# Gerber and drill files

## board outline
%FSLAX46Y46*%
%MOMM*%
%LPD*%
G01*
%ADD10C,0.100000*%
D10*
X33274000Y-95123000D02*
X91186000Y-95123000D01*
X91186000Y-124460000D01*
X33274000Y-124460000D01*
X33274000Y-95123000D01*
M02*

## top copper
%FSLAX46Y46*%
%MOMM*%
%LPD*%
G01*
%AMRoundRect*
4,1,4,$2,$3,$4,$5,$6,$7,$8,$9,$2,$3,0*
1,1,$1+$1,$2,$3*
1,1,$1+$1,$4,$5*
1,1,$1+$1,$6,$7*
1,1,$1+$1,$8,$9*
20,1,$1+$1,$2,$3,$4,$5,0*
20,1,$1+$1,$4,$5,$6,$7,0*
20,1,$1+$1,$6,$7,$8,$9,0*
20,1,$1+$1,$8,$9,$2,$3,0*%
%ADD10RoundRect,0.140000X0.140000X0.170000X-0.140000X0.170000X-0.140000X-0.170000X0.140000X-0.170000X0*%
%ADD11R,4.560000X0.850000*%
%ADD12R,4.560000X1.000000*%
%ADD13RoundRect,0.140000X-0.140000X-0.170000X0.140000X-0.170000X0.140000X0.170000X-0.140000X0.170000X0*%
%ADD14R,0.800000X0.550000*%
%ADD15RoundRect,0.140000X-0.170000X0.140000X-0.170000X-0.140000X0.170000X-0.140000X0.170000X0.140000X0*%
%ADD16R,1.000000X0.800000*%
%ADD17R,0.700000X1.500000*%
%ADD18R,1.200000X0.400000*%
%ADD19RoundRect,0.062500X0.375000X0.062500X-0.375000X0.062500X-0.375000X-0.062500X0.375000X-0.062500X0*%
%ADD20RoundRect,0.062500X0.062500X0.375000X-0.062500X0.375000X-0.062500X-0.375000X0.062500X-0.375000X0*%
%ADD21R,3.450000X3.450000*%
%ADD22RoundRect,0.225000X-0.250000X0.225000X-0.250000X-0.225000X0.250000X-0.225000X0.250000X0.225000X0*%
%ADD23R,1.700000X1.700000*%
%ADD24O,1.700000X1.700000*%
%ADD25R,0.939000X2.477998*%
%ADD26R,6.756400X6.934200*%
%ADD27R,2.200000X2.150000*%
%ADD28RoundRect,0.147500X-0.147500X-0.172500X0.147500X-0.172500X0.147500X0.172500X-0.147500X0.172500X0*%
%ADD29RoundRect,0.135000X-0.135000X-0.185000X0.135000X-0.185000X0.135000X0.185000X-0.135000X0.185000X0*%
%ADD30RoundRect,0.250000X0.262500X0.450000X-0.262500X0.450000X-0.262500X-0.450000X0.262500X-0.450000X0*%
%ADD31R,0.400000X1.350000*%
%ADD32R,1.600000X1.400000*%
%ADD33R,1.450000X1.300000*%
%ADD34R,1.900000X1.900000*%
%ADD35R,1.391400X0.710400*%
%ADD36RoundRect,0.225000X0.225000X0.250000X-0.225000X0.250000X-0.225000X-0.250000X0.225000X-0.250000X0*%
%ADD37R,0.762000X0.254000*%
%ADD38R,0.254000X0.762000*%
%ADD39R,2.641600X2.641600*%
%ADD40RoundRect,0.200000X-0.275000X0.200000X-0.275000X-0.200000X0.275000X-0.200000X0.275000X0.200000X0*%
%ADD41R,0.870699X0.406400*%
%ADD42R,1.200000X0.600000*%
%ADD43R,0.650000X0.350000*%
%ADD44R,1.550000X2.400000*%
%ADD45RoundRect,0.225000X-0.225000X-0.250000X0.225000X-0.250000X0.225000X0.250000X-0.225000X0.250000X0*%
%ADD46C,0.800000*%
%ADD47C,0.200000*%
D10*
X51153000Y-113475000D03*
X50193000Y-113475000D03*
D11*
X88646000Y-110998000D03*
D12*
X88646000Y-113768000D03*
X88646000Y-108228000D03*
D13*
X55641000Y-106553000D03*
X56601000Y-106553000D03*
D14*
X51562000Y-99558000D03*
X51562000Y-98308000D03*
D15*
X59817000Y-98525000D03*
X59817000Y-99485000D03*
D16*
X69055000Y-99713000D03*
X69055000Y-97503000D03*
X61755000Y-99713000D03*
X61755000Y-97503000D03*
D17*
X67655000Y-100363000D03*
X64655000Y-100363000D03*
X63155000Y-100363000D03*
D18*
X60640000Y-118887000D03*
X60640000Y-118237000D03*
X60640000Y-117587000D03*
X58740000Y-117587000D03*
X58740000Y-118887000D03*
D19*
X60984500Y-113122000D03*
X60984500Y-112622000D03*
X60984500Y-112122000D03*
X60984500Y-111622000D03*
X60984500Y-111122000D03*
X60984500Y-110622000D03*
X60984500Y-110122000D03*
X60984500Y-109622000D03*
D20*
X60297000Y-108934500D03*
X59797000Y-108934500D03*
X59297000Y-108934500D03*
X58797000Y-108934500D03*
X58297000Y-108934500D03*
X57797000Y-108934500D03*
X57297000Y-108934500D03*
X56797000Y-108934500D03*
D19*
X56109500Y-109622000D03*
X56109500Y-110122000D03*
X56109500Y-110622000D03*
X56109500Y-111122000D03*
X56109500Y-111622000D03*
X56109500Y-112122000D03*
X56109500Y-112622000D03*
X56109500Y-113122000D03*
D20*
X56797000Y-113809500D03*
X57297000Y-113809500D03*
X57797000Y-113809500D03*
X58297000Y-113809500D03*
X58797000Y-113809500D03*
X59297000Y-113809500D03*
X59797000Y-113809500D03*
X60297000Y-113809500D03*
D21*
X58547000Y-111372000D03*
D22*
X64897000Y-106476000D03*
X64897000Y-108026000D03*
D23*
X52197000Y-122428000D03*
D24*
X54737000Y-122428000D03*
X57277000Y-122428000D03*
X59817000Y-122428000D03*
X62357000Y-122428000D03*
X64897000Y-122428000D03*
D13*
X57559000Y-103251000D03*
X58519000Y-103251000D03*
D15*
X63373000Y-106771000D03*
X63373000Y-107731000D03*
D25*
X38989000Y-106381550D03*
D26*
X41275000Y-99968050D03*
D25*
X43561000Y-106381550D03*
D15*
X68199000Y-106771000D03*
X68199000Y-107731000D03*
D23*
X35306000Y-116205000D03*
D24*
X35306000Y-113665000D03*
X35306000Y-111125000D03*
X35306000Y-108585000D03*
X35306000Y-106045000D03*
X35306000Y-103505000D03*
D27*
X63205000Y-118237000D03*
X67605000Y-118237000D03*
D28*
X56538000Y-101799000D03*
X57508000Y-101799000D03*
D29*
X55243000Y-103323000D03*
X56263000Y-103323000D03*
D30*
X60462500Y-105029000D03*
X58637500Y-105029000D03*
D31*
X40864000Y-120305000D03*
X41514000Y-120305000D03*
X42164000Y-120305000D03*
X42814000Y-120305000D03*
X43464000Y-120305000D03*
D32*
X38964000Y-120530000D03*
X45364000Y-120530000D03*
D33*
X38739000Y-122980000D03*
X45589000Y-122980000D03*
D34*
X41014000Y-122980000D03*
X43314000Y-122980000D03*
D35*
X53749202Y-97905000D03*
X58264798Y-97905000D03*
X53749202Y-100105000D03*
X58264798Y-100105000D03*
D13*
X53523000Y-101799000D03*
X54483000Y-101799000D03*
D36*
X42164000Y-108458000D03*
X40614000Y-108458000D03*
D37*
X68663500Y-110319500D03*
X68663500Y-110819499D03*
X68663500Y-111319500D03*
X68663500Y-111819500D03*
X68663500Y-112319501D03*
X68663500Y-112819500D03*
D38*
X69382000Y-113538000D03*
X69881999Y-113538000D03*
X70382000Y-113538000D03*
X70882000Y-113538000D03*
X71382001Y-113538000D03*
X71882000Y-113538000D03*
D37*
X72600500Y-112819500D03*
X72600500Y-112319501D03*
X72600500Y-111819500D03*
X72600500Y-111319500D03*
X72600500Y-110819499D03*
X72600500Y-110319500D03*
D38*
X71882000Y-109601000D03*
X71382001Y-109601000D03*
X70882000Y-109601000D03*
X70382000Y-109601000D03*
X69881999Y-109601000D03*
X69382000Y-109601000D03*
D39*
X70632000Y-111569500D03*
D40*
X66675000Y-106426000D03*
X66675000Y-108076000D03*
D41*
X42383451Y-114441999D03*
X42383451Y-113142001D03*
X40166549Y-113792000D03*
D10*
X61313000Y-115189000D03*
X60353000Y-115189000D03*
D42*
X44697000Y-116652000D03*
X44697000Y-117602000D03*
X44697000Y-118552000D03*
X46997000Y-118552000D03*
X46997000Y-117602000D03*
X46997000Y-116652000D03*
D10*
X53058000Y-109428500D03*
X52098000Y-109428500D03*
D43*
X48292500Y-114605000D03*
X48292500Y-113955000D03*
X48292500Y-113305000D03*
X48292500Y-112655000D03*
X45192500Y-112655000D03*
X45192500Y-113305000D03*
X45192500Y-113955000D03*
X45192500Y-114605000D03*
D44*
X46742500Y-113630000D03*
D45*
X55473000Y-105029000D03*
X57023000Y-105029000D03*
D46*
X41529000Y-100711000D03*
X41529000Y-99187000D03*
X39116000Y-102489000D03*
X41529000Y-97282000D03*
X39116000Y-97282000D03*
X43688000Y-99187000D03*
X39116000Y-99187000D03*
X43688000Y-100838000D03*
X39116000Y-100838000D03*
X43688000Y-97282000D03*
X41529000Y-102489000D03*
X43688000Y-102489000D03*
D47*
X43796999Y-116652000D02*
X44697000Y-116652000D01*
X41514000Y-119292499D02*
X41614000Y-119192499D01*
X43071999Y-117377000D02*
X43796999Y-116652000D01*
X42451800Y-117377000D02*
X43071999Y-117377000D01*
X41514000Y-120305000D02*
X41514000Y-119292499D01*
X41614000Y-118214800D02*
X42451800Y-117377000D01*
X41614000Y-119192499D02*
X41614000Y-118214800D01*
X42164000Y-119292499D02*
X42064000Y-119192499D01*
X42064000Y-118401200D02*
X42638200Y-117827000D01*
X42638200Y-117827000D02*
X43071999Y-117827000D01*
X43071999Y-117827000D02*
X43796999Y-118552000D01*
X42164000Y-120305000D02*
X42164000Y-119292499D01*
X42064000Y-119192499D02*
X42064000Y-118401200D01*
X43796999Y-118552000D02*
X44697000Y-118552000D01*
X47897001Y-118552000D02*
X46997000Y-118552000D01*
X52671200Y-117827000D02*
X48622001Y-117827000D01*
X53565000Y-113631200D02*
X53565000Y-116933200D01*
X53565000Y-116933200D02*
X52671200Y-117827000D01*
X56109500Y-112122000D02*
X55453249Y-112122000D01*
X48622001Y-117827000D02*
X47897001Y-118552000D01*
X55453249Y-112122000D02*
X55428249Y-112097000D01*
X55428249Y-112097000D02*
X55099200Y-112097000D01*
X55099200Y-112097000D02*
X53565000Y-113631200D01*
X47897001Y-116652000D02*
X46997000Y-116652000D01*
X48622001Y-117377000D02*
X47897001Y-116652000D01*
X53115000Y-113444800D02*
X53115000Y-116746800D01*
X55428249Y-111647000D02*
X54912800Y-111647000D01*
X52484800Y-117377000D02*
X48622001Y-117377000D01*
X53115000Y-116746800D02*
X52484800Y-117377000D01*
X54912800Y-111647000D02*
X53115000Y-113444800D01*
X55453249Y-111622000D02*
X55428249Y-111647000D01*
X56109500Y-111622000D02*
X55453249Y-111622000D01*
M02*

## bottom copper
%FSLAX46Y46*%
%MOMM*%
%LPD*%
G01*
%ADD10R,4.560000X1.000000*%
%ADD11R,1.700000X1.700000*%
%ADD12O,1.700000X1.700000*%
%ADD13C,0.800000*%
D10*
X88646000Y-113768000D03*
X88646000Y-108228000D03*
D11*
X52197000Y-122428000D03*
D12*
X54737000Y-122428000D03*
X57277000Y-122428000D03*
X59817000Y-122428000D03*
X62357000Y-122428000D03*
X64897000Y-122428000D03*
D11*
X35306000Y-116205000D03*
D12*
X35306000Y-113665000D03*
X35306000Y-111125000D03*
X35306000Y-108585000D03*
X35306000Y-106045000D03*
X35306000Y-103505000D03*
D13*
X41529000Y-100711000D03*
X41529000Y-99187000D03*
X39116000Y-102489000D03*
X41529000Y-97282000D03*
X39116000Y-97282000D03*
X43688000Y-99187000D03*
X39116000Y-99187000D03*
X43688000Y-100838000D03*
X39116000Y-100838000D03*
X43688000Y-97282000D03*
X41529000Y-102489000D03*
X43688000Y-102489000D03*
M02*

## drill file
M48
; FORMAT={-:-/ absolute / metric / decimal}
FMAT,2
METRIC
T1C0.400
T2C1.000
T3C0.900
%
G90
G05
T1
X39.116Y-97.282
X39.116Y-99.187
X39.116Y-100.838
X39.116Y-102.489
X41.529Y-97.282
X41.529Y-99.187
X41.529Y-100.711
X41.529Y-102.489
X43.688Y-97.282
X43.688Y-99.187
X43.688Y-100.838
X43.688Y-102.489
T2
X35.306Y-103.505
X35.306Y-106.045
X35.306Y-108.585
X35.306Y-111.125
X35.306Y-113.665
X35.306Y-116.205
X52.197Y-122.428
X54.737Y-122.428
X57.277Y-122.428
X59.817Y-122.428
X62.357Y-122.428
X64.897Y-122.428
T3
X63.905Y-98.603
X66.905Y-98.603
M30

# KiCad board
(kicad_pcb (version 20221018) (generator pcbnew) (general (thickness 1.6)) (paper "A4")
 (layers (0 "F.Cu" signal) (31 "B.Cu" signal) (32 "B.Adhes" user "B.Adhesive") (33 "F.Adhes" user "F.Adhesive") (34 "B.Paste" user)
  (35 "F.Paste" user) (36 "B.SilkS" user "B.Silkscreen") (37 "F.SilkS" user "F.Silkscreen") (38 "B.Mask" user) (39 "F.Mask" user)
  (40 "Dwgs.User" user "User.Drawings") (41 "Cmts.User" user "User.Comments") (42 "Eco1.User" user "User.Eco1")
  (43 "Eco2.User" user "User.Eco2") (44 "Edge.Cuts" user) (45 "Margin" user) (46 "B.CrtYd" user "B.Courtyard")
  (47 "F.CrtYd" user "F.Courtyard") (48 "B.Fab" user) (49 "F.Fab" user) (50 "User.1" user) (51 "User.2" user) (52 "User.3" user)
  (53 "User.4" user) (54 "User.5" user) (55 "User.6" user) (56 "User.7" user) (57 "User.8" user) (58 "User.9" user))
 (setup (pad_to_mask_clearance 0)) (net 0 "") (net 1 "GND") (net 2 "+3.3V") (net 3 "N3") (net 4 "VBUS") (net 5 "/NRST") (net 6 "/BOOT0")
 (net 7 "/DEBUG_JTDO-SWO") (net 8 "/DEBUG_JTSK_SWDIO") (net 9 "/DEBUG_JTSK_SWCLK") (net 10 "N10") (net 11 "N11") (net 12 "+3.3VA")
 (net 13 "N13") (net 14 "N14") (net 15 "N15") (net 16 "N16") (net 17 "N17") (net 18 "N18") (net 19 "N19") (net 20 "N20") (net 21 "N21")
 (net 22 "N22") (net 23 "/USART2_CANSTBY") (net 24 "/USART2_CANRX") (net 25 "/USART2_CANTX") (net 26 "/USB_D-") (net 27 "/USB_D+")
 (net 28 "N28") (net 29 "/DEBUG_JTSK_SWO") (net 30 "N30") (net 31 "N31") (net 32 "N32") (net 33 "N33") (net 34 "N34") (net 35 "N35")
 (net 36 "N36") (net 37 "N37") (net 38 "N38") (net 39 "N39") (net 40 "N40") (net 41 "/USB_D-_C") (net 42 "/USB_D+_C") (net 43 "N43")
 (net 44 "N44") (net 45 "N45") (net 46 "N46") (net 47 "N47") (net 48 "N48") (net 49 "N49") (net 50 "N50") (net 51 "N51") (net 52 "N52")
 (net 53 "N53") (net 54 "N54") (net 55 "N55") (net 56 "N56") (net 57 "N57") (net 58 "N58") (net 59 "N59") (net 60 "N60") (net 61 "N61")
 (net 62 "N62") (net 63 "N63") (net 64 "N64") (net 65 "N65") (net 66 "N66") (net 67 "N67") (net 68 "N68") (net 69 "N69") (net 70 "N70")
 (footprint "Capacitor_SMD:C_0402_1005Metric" (layer "F.Cu") (at 50.673 113.475 180)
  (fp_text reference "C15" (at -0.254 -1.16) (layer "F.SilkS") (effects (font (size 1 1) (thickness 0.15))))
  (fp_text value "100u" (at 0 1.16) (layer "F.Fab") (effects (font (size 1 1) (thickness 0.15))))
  (pad "1" smd roundrect (at -0.48 0 180) (size 0.56 0.62) (layers "F.Cu" "F.Paste" "F.Mask") (roundrect_rratio 0.25) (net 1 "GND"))
  (pad "2" smd roundrect (at 0.48 0 180) (size 0.56 0.62) (layers "F.Cu" "F.Paste" "F.Mask") (roundrect_rratio 0.25) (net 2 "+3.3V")))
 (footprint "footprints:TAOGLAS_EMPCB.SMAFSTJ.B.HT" (layer "F.Cu") (at 88.646 110.998 90)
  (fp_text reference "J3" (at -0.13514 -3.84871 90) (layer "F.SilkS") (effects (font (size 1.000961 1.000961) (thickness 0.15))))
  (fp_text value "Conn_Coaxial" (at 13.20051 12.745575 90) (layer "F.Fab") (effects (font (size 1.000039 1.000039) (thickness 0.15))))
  (pad "1" smd rect (at 0 0 90) (size 0.85 4.56) (layers "F.Cu" "F.Paste" "F.Mask") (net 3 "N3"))
  (pad "SH1" smd rect (at -2.77 0 90) (size 1 4.56) (layers "F.Cu" "F.Paste" "F.Mask"))
  (pad "SH2" smd rect (at 2.77 0 90) (size 1 4.56) (layers "F.Cu" "F.Paste" "F.Mask"))
  (pad "SH3" smd rect (at -2.77 0 90) (size 1 4.56) (layers "B.Cu" "B.Paste" "B.Mask"))
  (pad "SH4" smd rect (at 2.77 0 90) (size 1 4.56) (layers "B.Cu" "B.Paste" "B.Mask")))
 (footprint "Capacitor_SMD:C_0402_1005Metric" (layer "F.Cu") (at 56.121 106.553)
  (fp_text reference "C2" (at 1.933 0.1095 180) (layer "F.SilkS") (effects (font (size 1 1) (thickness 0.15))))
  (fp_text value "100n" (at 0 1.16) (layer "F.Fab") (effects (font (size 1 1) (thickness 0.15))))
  (pad "1" smd roundrect (at -0.48 0) (size 0.56 0.62) (layers "F.Cu" "F.Paste" "F.Mask") (roundrect_rratio 0.25) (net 2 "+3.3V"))
  (pad "2" smd roundrect (at 0.48 0) (size 0.56 0.62) (layers "F.Cu" "F.Paste" "F.Mask") (roundrect_rratio 0.25) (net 1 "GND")))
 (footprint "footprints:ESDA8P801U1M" (layer "F.Cu") (at 51.562 98.933 90)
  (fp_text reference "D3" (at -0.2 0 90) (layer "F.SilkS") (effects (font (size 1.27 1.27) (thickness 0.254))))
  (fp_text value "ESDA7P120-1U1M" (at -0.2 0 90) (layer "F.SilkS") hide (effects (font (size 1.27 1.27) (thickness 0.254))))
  (pad "1" smd rect (at -0.625 0 90) (size 0.55 0.8) (layers "F.Cu" "F.Paste" "F.Mask") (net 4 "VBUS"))
  (pad "2" smd rect (at 0.625 0 90) (size 0.55 0.8) (layers "F.Cu" "F.Paste" "F.Mask") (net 1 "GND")))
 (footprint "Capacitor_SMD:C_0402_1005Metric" (layer "F.Cu") (at 59.817 99.005 -90)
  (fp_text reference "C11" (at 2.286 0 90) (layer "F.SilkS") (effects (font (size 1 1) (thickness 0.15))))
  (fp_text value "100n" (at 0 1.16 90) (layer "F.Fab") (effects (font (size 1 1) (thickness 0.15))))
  (pad "1" smd roundrect (at -0.48 0 270) (size 0.56 0.62) (layers "F.Cu" "F.Paste" "F.Mask") (roundrect_rratio 0.25) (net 1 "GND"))
  (pad "2" smd roundrect (at 0.48 0 270) (size 0.56 0.62) (layers "F.Cu" "F.Paste" "F.Mask") (roundrect_rratio 0.25) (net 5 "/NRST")))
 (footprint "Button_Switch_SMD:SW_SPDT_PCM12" (layer "F.Cu") (at 65.405 98.933 180)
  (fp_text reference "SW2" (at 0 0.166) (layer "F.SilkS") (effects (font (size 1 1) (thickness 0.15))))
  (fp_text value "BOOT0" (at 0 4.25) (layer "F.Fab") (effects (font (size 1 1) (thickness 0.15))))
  (pad "" smd rect (at -3.65 -0.78 180) (size 1 0.8) (layers "F.Cu" "F.Paste" "F.Mask"))
  (pad "" smd rect (at -3.65 1.43 180) (size 1 0.8) (layers "F.Cu" "F.Paste" "F.Mask"))
  (pad "" np_thru_hole circle (at -1.5 0.33 180) (size 0.9 0.9) (drill 0.9) (layers "*.Cu" "*.Mask"))
  (pad "" np_thru_hole circle (at 1.5 0.33 180) (size 0.9 0.9) (drill 0.9) (layers "*.Cu" "*.Mask"))
  (pad "" smd rect (at 3.65 -0.78 180) (size 1 0.8) (layers "F.Cu" "F.Paste" "F.Mask"))
  (pad "" smd rect (at 3.65 1.43 180) (size 1 0.8) (layers "F.Cu" "F.Paste" "F.Mask"))
  (pad "1" smd rect (at -2.25 -1.43 180) (size 0.7 1.5) (layers "F.Cu" "F.Paste" "F.Mask") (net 1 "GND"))
  (pad "2" smd rect (at 0.75 -1.43 180) (size 0.7 1.5) (layers "F.Cu" "F.Paste" "F.Mask") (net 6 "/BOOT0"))
  (pad "3" smd rect (at 2.25 -1.43 180) (size 0.7 1.5) (layers "F.Cu" "F.Paste" "F.Mask") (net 2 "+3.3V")))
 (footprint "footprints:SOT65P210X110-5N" (layer "F.Cu") (at 59.69 118.237 180)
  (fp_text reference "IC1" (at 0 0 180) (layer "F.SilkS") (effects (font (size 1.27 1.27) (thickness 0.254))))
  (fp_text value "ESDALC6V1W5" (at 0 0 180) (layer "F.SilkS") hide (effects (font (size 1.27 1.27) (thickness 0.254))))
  (pad "1" smd rect (at -0.95 -0.65 270) (size 0.4 1.2) (layers "F.Cu" "F.Paste" "F.Mask") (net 5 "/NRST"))
  (pad "2" smd rect (at -0.95 0 270) (size 0.4 1.2) (layers "F.Cu" "F.Paste" "F.Mask") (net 1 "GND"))
  (pad "3" smd rect (at -0.95 0.65 270) (size 0.4 1.2) (layers "F.Cu" "F.Paste" "F.Mask") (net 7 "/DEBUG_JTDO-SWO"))
  (pad "4" smd rect (at 0.95 0.65 270) (size 0.4 1.2) (layers "F.Cu" "F.Paste" "F.Mask") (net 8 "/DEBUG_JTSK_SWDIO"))
  (pad "5" smd rect (at 0.95 -0.65 270) (size 0.4 1.2) (layers "F.Cu" "F.Paste" "F.Mask") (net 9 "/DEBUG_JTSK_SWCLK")))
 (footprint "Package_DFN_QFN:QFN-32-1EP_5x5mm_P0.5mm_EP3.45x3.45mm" (layer "F.Cu") (at 58.547 111.372 180)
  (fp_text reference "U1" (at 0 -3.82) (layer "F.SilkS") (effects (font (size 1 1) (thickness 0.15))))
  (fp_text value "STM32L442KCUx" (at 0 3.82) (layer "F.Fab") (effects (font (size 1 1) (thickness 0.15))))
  (pad "" smd roundrect (at -1.15 -1.15 180) (size 0.93 0.93) (layers "F.Paste") (roundrect_rratio 0.25))
  (pad "" smd roundrect (at -1.15 0 180) (size 0.93 0.93) (layers "F.Paste") (roundrect_rratio 0.25))
  (pad "" smd roundrect (at -1.15 1.15 180) (size 0.93 0.93) (layers "F.Paste") (roundrect_rratio 0.25))
  (pad "" smd roundrect (at 0 -1.15 180) (size 0.93 0.93) (layers "F.Paste") (roundrect_rratio 0.25))
  (pad "" smd roundrect (at 0 0 180) (size 0.93 0.93) (layers "F.Paste") (roundrect_rratio 0.25))
  (pad "" smd roundrect (at 0 1.15 180) (size 0.93 0.93) (layers "F.Paste") (roundrect_rratio 0.25))
  (pad "" smd roundrect (at 1.15 -1.15 180) (size 0.93 0.93) (layers "F.Paste") (roundrect_rratio 0.25))
  (pad "" smd roundrect (at 1.15 0 180) (size 0.93 0.93) (layers "F.Paste") (roundrect_rratio 0.25))
  (pad "" smd roundrect (at 1.15 1.15 180) (size 0.93 0.93) (layers "F.Paste") (roundrect_rratio 0.25))
  (pad "1" smd roundrect (at -2.4375 -1.75 180) (size 0.875 0.25) (layers "F.Cu" "F.Paste" "F.Mask") (roundrect_rratio 0.25) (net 2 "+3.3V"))
  (pad "2" smd roundrect (at -2.4375 -1.25 180) (size 0.875 0.25) (layers "F.Cu" "F.Paste" "F.Mask") (roundrect_rratio 0.25) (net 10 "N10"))
  (pad "3" smd roundrect (at -2.4375 -0.75 180) (size 0.875 0.25) (layers "F.Cu" "F.Paste" "F.Mask") (roundrect_rratio 0.25) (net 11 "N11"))
  (pad "4" smd roundrect (at -2.4375 -0.25 180) (size 0.875 0.25) (layers "F.Cu" "F.Paste" "F.Mask") (roundrect_rratio 0.25) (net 5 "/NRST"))
  (pad "5" smd roundrect (at -2.4375 0.25 180) (size 0.875 0.25) (layers "F.Cu" "F.Paste" "F.Mask") (roundrect_rratio 0.25)
   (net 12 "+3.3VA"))
  (pad "6" smd roundrect (at -2.4375 0.75 180) (size 0.875 0.25) (layers "F.Cu" "F.Paste" "F.Mask") (roundrect_rratio 0.25) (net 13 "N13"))
  (pad "7" smd roundrect (at -2.4375 1.25 180) (size 0.875 0.25) (layers "F.Cu" "F.Paste" "F.Mask") (roundrect_rratio 0.25) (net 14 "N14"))
  (pad "8" smd roundrect (at -2.4375 1.75 180) (size 0.875 0.25) (layers "F.Cu" "F.Paste" "F.Mask") (roundrect_rratio 0.25) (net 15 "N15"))
  (pad "9" smd roundrect (at -1.75 2.4375 180) (size 0.25 0.875) (layers "F.Cu" "F.Paste" "F.Mask") (roundrect_rratio 0.25) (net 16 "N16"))
  (pad "10" smd roundrect (at -1.25 2.4375 180) (size 0.25 0.875) (layers "F.Cu" "F.Paste" "F.Mask") (roundrect_rratio 0.25) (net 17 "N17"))
  (pad "11" smd roundrect (at -0.75 2.4375 180) (size 0.25 0.875) (layers "F.Cu" "F.Paste" "F.Mask") (roundrect_rratio 0.25) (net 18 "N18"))
  (pad "12" smd roundrect (at -0.25 2.4375 180) (size 0.25 0.875) (layers "F.Cu" "F.Paste" "F.Mask") (roundrect_rratio 0.25) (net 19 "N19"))
  (pad "13" smd roundrect (at 0.25 2.4375 180) (size 0.25 0.875) (layers "F.Cu" "F.Paste" "F.Mask") (roundrect_rratio 0.25) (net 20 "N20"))
  (pad "14" smd roundrect (at 0.75 2.4375 180) (size 0.25 0.875) (layers "F.Cu" "F.Paste" "F.Mask") (roundrect_rratio 0.25) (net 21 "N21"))
  (pad "15" smd roundrect (at 1.25 2.4375 180) (size 0.25 0.875) (layers "F.Cu" "F.Paste" "F.Mask") (roundrect_rratio 0.25) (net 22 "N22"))
  (pad "16" smd roundrect (at 1.75 2.4375 180) (size 0.25 0.875) (layers "F.Cu" "F.Paste" "F.Mask") (roundrect_rratio 0.25) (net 1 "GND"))
  (pad "17" smd roundrect (at 2.4375 1.75 180) (size 0.875 0.25) (layers "F.Cu" "F.Paste" "F.Mask") (roundrect_rratio 0.25) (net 2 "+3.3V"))
  (pad "18" smd roundrect (at 2.4375 1.25 180) (size 0.875 0.25) (layers "F.Cu" "F.Paste" "F.Mask") (roundrect_rratio 0.25)
   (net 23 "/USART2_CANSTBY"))
  (pad "19" smd roundrect (at 2.4375 0.75 180) (size 0.875 0.25) (layers "F.Cu" "F.Paste" "F.Mask") (roundrect_rratio 0.25)
   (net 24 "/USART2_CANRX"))
  (pad "20" smd roundrect (at 2.4375 0.25 180) (size 0.875 0.25) (layers "F.Cu" "F.Paste" "F.Mask") (roundrect_rratio 0.25)
   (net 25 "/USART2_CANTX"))
  (pad "21" smd roundrect (at 2.4375 -0.25 180) (size 0.875 0.25) (layers "F.Cu" "F.Paste" "F.Mask") (roundrect_rratio 0.25)
   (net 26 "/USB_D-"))
  (pad "22" smd roundrect (at 2.4375 -0.75 180) (size 0.875 0.25) (layers "F.Cu" "F.Paste" "F.Mask") (roundrect_rratio 0.25)
   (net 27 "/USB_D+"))
  (pad "23" smd roundrect (at 2.4375 -1.25 180) (size 0.875 0.25) (layers "F.Cu" "F.Paste" "F.Mask") (roundrect_rratio 0.25)
   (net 8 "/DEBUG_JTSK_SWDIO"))
  (pad "24" smd roundrect (at 2.4375 -1.75 180) (size 0.875 0.25) (layers "F.Cu" "F.Paste" "F.Mask") (roundrect_rratio 0.25)
   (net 9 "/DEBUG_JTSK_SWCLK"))
  (pad "25" smd roundrect (at 1.75 -2.4375 180) (size 0.25 0.875) (layers "F.Cu" "F.Paste" "F.Mask") (roundrect_rratio 0.25) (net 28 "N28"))
  (pad "26" smd roundrect (at 1.25 -2.4375 180) (size 0.25 0.875) (layers "F.Cu" "F.Paste" "F.Mask") (roundrect_rratio 0.25)
   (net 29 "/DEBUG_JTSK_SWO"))
  (pad "27" smd roundrect (at 0.75 -2.4375 180) (size 0.25 0.875) (layers "F.Cu" "F.Paste" "F.Mask") (roundrect_rratio 0.25) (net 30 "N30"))
  (pad "28" smd roundrect (at 0.25 -2.4375 180) (size 0.25 0.875) (layers "F.Cu" "F.Paste" "F.Mask") (roundrect_rratio 0.25) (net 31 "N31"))
  (pad "29" smd roundrect (at -0.25 -2.4375 180) (size 0.25 0.875) (layers "F.Cu" "F.Paste" "F.Mask") (roundrect_rratio 0.25) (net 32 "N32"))
  (pad "30" smd roundrect (at -0.75 -2.4375 180) (size 0.25 0.875) (layers "F.Cu" "F.Paste" "F.Mask") (roundrect_rratio 0.25) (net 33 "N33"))
  (pad "31" smd roundrect (at -1.25 -2.4375 180) (size 0.25 0.875) (layers "F.Cu" "F.Paste" "F.Mask") (roundrect_rratio 0.25)
   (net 6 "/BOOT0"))
  (pad "32" smd roundrect (at -1.75 -2.4375 180) (size 0.25 0.875) (layers "F.Cu" "F.Paste" "F.Mask") (roundrect_rratio 0.25) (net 1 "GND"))
  (pad "33" smd rect (at 0 0 180) (size 3.45 3.45) (layers "F.Cu" "F.Mask") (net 1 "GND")))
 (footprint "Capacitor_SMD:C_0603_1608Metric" (layer "F.Cu") (at 64.897 107.251 -90)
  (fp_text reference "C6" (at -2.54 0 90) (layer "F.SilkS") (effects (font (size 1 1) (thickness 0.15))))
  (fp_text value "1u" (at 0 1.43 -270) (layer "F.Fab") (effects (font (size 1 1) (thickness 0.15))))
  (pad "1" smd roundrect (at -0.775 0 270) (size 0.9 0.95) (layers "F.Cu" "F.Paste" "F.Mask") (roundrect_rratio 0.25) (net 12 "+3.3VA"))
  (pad "2" smd roundrect (at 0.775 0 270) (size 0.9 0.95) (layers "F.Cu" "F.Paste" "F.Mask") (roundrect_rratio 0.25) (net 1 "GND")))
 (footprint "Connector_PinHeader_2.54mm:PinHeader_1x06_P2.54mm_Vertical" (layer "F.Cu") (at 52.197 122.428 90)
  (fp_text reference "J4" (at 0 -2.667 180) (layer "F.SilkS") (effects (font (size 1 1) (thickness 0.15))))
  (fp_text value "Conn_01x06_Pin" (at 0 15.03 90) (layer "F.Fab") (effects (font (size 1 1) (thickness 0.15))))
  (pad "1" thru_hole rect (at 0 0 90) (size 1.7 1.7) (drill 1) (layers "*.Cu" "*.Mask") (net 2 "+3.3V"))
  (pad "2" thru_hole oval (at 0 2.54 90) (size 1.7 1.7) (drill 1) (layers "*.Cu" "*.Mask") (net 9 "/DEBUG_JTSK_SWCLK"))
  (pad "3" thru_hole oval (at 0 5.08 90) (size 1.7 1.7) (drill 1) (layers "*.Cu" "*.Mask") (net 1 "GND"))
  (pad "4" thru_hole oval (at 0 7.62 90) (size 1.7 1.7) (drill 1) (layers "*.Cu" "*.Mask") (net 8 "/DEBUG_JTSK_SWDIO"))
  (pad "5" thru_hole oval (at 0 10.16 90) (size 1.7 1.7) (drill 1) (layers "*.Cu" "*.Mask") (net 5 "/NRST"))
  (pad "6" thru_hole oval (at 0 12.7 90) (size 1.7 1.7) (drill 1) (layers "*.Cu" "*.Mask") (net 7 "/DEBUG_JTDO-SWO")))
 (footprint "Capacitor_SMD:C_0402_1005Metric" (layer "F.Cu") (at 58.039 103.251)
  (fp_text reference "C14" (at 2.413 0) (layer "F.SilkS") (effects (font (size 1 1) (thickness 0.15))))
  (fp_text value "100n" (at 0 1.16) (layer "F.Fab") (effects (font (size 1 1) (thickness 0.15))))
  (pad "1" smd roundrect (at -0.48 0) (size 0.56 0.62) (layers "F.Cu" "F.Paste" "F.Mask") (roundrect_rratio 0.25) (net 1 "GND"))
  (pad "2" smd roundrect (at 0.48 0) (size 0.56 0.62) (layers "F.Cu" "F.Paste" "F.Mask") (roundrect_rratio 0.25) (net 4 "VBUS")))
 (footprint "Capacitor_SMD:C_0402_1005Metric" (layer "F.Cu") (at 63.373 107.251 -90)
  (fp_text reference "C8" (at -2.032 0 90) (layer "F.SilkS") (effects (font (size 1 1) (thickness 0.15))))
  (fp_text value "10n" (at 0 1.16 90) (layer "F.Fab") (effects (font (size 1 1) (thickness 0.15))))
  (pad "1" smd roundrect (at -0.48 0 270) (size 0.56 0.62) (layers "F.Cu" "F.Paste" "F.Mask") (roundrect_rratio 0.25) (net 12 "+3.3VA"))
  (pad "2" smd roundrect (at 0.48 0 270) (size 0.56 0.62) (layers "F.Cu" "F.Paste" "F.Mask") (roundrect_rratio 0.25) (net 1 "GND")))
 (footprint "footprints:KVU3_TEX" (layer "F.Cu") (at 41.275 99.96805)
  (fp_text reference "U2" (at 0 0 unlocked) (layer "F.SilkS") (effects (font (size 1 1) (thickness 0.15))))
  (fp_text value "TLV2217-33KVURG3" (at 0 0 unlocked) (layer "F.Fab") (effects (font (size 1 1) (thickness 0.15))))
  (pad "1" smd rect (at -2.286 6.4135) (size 0.939 2.477998) (layers "F.Cu" "F.Paste" "F.Mask") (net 2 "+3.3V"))
  (pad "2" smd rect (at 0 0) (size 6.7564 6.9342) (layers "F.Cu" "F.Paste" "F.Mask") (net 1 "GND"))
  (pad "3" smd rect (at 2.286 6.4135) (size 0.939 2.477998) (layers "F.Cu" "F.Paste" "F.Mask") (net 4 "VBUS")))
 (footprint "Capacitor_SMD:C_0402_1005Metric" (layer "F.Cu") (at 68.199 107.251 -90)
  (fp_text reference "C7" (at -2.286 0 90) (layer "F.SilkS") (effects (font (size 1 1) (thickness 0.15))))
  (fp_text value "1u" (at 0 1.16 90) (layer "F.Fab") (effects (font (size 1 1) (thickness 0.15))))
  (pad "1" smd roundrect (at -0.48 0 270) (size 0.56 0.62) (layers "F.Cu" "F.Paste" "F.Mask") (roundrect_rratio 0.25) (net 2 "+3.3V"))
  (pad "2" smd roundrect (at 0.48 0 270) (size 0.56 0.62) (layers "F.Cu" "F.Paste" "F.Mask") (roundrect_rratio 0.25) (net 1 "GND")))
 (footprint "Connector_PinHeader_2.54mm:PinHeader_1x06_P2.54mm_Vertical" (layer "F.Cu") (at 35.306 116.205 180)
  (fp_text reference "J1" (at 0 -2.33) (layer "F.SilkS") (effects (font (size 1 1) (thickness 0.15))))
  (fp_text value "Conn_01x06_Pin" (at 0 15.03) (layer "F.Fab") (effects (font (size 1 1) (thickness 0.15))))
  (pad "1" thru_hole rect (at 0 0 180) (size 1.7 1.7) (drill 1) (layers "*.Cu" "*.Mask") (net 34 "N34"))
  (pad "2" thru_hole oval (at 0 2.54 180) (size 1.7 1.7) (drill 1) (layers "*.Cu" "*.Mask") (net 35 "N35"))
  (pad "3" thru_hole oval (at 0 5.08 180) (size 1.7 1.7) (drill 1) (layers "*.Cu" "*.Mask") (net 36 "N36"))
  (pad "4" thru_hole oval (at 0 7.62 180) (size 1.7 1.7) (drill 1) (layers "*.Cu" "*.Mask") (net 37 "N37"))
  (pad "5" thru_hole oval (at 0 10.16 180) (size 1.7 1.7) (drill 1) (layers "*.Cu" "*.Mask") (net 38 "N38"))
  (pad "6" thru_hole oval (at 0 12.7 180) (size 1.7 1.7) (drill 1) (layers "*.Cu" "*.Mask") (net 1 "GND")))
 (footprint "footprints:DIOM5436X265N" (layer "F.Cu") (at 65.405 118.237)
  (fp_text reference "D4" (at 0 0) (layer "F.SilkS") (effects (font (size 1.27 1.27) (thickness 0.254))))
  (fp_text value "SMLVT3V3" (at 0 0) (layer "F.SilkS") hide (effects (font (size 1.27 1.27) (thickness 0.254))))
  (pad "1" smd rect (at -2.2 0 90) (size 2.15 2.2) (layers "F.Cu" "F.Paste" "F.Mask") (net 2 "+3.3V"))
  (pad "2" smd rect (at 2.2 0 90) (size 2.15 2.2) (layers "F.Cu" "F.Paste" "F.Mask") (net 1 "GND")))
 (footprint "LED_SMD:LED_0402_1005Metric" (layer "F.Cu") (at 57.023 101.799)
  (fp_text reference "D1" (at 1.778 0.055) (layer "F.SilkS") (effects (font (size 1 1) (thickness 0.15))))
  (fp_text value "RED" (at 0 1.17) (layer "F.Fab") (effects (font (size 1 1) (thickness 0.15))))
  (pad "1" smd roundrect (at -0.485 0) (size 0.59 0.64) (layers "F.Cu" "F.Paste" "F.Mask") (roundrect_rratio 0.25) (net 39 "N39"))
  (pad "2" smd roundrect (at 0.485 0) (size 0.59 0.64) (layers "F.Cu" "F.Paste" "F.Mask") (roundrect_rratio 0.25) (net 4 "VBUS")))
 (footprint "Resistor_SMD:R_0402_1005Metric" (layer "F.Cu") (at 55.753 103.323)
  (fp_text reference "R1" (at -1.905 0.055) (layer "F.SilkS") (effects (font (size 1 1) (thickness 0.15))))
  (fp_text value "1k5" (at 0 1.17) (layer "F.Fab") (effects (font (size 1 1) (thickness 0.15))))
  (pad "1" smd roundrect (at -0.51 0) (size 0.54 0.64) (layers "F.Cu" "F.Paste" "F.Mask") (roundrect_rratio 0.25) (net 1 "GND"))
  (pad "2" smd roundrect (at 0.51 0) (size 0.54 0.64) (layers "F.Cu" "F.Paste" "F.Mask") (roundrect_rratio 0.25) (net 39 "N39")))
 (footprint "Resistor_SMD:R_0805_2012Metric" (layer "F.Cu") (at 59.55 105.029 180)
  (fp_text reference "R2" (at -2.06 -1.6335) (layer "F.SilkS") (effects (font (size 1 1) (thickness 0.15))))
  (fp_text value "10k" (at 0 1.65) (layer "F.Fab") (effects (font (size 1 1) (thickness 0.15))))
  (pad "1" smd roundrect (at -0.9125 0 180) (size 1.025 1.4) (layers "F.Cu" "F.Paste" "F.Mask") (roundrect_rratio 0.243902439)
   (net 6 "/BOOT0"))
  (pad "2" smd roundrect (at 0.9125 0 180) (size 1.025 1.4) (layers "F.Cu" "F.Paste" "F.Mask") (roundrect_rratio 0.243902439)
   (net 6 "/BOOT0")))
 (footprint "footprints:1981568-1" (layer "F.Cu") (at 42.164 125.73)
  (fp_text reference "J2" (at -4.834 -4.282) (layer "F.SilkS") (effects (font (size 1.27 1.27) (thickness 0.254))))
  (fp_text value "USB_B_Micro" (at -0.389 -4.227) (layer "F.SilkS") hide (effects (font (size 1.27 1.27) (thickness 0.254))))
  (pad "1" smd rect (at -1.3 -5.425) (size 0.4 1.35) (layers "F.Cu" "F.Paste" "F.Mask") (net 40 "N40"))
  (pad "2" smd rect (at -0.65 -5.425) (size 0.4 1.35) (layers "F.Cu" "F.Paste" "F.Mask") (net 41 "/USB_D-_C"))
  (pad "3" smd rect (at 0 -5.425) (size 0.4 1.35) (layers "F.Cu" "F.Paste" "F.Mask") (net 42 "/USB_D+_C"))
  (pad "4" smd rect (at 0.65 -5.425) (size 0.4 1.35) (layers "F.Cu" "F.Paste" "F.Mask") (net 4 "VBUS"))
  (pad "5" smd rect (at 1.3 -5.425) (size 0.4 1.35) (layers "F.Cu" "F.Paste" "F.Mask") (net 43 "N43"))
  (pad "6" smd rect (at -3.2 -5.2 90) (size 1.4 1.6) (layers "F.Cu" "F.Paste" "F.Mask") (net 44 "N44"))
  (pad "7" smd rect (at 3.2 -5.2 90) (size 1.4 1.6) (layers "F.Cu" "F.Paste" "F.Mask"))
  (pad "8" smd rect (at -3.425 -2.75 90) (size 1.3 1.45) (layers "F.Cu" "F.Paste" "F.Mask"))
  (pad "9" smd rect (at 3.425 -2.75 90) (size 1.3 1.45) (layers "F.Cu" "F.Paste" "F.Mask"))
  (pad "10" smd rect (at -1.15 -2.75 90) (size 1.9 1.9) (layers "F.Cu" "F.Paste" "F.Mask"))
  (pad "11" smd rect (at 1.15 -2.75 90) (size 1.9 1.9) (layers "F.Cu" "F.Paste" "F.Mask")))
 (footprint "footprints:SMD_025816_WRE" (layer "F.Cu") (at 56.007 99.005)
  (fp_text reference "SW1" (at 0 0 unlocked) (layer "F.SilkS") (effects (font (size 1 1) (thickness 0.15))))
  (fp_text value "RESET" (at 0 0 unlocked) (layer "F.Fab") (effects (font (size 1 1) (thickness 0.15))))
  (pad "1" smd rect (at -2.257798 -1.1) (size 1.3914 0.7104) (layers "F.Cu" "F.Paste" "F.Mask") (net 1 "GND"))
  (pad "2" smd rect (at 2.257798 -1.1) (size 1.3914 0.7104) (layers "F.Cu" "F.Paste" "F.Mask") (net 1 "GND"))
  (pad "3" smd rect (at -2.257798 1.1) (size 1.3914 0.7104) (layers "F.Cu" "F.Paste" "F.Mask") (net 5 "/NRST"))
  (pad "4" smd rect (at 2.257798 1.1) (size 1.3914 0.7104) (layers "F.Cu" "F.Paste" "F.Mask") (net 5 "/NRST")))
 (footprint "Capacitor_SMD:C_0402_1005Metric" (layer "F.Cu") (at 54.003 101.799)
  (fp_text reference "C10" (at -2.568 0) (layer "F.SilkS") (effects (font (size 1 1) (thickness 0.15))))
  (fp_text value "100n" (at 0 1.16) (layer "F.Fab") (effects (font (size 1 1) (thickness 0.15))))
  (pad "1" smd roundrect (at -0.48 0) (size 0.56 0.62) (layers "F.Cu" "F.Paste" "F.Mask") (roundrect_rratio 0.25) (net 4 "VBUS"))
  (pad "2" smd roundrect (at 0.48 0) (size 0.56 0.62) (layers "F.Cu" "F.Paste" "F.Mask") (roundrect_rratio 0.25) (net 1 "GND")))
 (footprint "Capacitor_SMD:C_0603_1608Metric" (layer "F.Cu") (at 41.389 108.458 180)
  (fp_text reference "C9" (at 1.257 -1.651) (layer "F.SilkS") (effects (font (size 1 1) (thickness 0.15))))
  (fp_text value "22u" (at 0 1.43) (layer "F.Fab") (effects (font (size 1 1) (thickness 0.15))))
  (pad "1" smd roundrect (at -0.775 0 180) (size 0.9 0.95) (layers "F.Cu" "F.Paste" "F.Mask") (roundrect_rratio 0.25) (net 2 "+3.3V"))
  (pad "2" smd roundrect (at 0.775 0 180) (size 0.9 0.95) (layers "F.Cu" "F.Paste" "F.Mask") (roundrect_rratio 0.25) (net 1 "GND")))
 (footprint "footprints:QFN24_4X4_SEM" (layer "F.Cu") (at 70.632 111.5695)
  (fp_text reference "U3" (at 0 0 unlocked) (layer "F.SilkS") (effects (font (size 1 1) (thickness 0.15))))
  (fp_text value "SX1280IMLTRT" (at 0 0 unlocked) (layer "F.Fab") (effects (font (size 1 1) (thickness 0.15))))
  (pad "1" smd rect (at -1.9685 -1.25 90) (size 0.254 0.762) (layers "F.Cu" "F.Paste" "F.Mask") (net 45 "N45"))
  (pad "2" smd rect (at -1.9685 -0.750001 90) (size 0.254 0.762) (layers "F.Cu" "F.Paste" "F.Mask") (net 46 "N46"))
  (pad "3" smd rect (at -1.9685 -0.25 90) (size 0.254 0.762) (layers "F.Cu" "F.Paste" "F.Mask") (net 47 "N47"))
  (pad "4" smd rect (at -1.9685 0.25 90) (size 0.254 0.762) (layers "F.Cu" "F.Paste" "F.Mask") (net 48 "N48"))
  (pad "5" smd rect (at -1.9685 0.750001 90) (size 0.254 0.762) (layers "F.Cu" "F.Paste" "F.Mask") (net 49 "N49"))
  (pad "6" smd rect (at -1.9685 1.25 90) (size 0.254 0.762) (layers "F.Cu" "F.Paste" "F.Mask") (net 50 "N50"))
  (pad "7" smd rect (at -1.25 1.9685) (size 0.254 0.762) (layers "F.Cu" "F.Paste" "F.Mask") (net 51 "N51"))
  (pad "8" smd rect (at -0.750001 1.9685) (size 0.254 0.762) (layers "F.Cu" "F.Paste" "F.Mask") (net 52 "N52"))
  (pad "9" smd rect (at -0.25 1.9685) (size 0.254 0.762) (layers "F.Cu" "F.Paste" "F.Mask") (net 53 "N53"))
  (pad "10" smd rect (at 0.25 1.9685) (size 0.254 0.762) (layers "F.Cu" "F.Paste" "F.Mask") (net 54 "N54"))
  (pad "11" smd rect (at 0.750001 1.9685) (size 0.254 0.762) (layers "F.Cu" "F.Paste" "F.Mask") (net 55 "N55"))
  (pad "12" smd rect (at 1.25 1.9685) (size 0.254 0.762) (layers "F.Cu" "F.Paste" "F.Mask") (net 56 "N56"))
  (pad "13" smd rect (at 1.9685 1.25 90) (size 0.254 0.762) (layers "F.Cu" "F.Paste" "F.Mask") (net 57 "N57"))
  (pad "14" smd rect (at 1.9685 0.750001 90) (size 0.254 0.762) (layers "F.Cu" "F.Paste" "F.Mask") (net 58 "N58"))
  (pad "15" smd rect (at 1.9685 0.25 90) (size 0.254 0.762) (layers "F.Cu" "F.Paste" "F.Mask") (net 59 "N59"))
  (pad "16" smd rect (at 1.9685 -0.25 90) (size 0.254 0.762) (layers "F.Cu" "F.Paste" "F.Mask") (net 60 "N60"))
  (pad "17" smd rect (at 1.9685 -0.750001 90) (size 0.254 0.762) (layers "F.Cu" "F.Paste" "F.Mask") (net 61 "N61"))
  (pad "18" smd rect (at 1.9685 -1.25 90) (size 0.254 0.762) (layers "F.Cu" "F.Paste" "F.Mask") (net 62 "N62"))
  (pad "19" smd rect (at 1.25 -1.9685) (size 0.254 0.762) (layers "F.Cu" "F.Paste" "F.Mask") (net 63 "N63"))
  (pad "20" smd rect (at 0.750001 -1.9685) (size 0.254 0.762) (layers "F.Cu" "F.Paste" "F.Mask") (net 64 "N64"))
  (pad "21" smd rect (at 0.25 -1.9685) (size 0.254 0.762) (layers "F.Cu" "F.Paste" "F.Mask") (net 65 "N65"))
  (pad "22" smd rect (at -0.25 -1.9685) (size 0.254 0.762) (layers "F.Cu" "F.Paste" "F.Mask") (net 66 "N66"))
  (pad "23" smd rect (at -0.750001 -1.9685) (size 0.254 0.762) (layers "F.Cu" "F.Paste" "F.Mask") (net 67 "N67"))
  (pad "24" smd rect (at -1.25 -1.9685) (size 0.254 0.762) (layers "F.Cu" "F.Paste" "F.Mask") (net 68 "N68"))
  (pad "25" smd rect (at 0 0) (size 2.6416 2.6416) (layers "F.Cu" "F.Paste" "F.Mask") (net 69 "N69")))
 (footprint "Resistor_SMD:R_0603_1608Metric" (layer "F.Cu") (at 66.675 107.251 -90)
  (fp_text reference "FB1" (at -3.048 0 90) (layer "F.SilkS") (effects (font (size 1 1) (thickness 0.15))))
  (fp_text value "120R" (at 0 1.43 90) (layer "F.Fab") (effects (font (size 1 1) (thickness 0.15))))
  (pad "1" smd roundrect (at -0.825 0 270) (size 0.8 0.95) (layers "F.Cu" "F.Paste" "F.Mask") (roundrect_rratio 0.25) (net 12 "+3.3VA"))
  (pad "2" smd roundrect (at 0.825 0 270) (size 0.8 0.95) (layers "F.Cu" "F.Paste" "F.Mask") (roundrect_rratio 0.25) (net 2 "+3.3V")))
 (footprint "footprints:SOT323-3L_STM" (layer "F.Cu") (at 41.275 113.792 180)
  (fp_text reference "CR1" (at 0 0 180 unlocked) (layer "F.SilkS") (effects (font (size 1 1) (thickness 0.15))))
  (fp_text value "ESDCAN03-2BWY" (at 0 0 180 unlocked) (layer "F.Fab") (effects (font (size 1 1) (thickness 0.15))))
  (pad "1" smd rect (at -1.108451 -0.649999 180) (size 0.870699 0.4064) (layers "F.Cu" "F.Paste" "F.Mask") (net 37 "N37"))
  (pad "2" smd rect (at -1.108451 0.649999 180) (size 0.870699 0.4064) (layers "F.Cu" "F.Paste" "F.Mask") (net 35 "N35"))
  (pad "3" smd rect (at 1.108451 0 180) (size 0.870699 0.4064) (layers "F.Cu" "F.Paste" "F.Mask") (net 1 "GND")))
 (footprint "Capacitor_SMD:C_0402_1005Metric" (layer "F.Cu") (at 60.833 115.189 180)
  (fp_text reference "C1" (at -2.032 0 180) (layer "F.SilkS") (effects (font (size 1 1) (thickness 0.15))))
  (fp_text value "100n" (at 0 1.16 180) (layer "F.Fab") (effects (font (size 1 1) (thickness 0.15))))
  (pad "1" smd roundrect (at -0.48 0 180) (size 0.56 0.62) (layers "F.Cu" "F.Paste" "F.Mask") (roundrect_rratio 0.25) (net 2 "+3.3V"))
  (pad "2" smd roundrect (at 0.48 0 180) (size 0.56 0.62) (layers "F.Cu" "F.Paste" "F.Mask") (roundrect_rratio 0.25) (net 1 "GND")))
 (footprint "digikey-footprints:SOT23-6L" (layer "F.Cu") (at 45.847 117.602 -90)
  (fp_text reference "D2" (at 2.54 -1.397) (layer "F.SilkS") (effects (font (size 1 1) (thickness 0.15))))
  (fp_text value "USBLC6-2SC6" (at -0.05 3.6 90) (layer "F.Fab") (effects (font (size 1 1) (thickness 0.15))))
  (pad "1" smd rect (at -0.95 1.15 270) (size 0.6 1.2) (layers "F.Cu" "F.Paste" "F.Mask") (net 41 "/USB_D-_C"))
  (pad "2" smd rect (at 0 1.15 270) (size 0.6 1.2) (layers "F.Cu" "F.Paste" "F.Mask") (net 1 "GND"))
  (pad "3" smd rect (at 0.95 1.15 270) (size 0.6 1.2) (layers "F.Cu" "F.Paste" "F.Mask") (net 42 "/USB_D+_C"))
  (pad "4" smd rect (at 0.95 -1.15 270) (size 0.6 1.2) (layers "F.Cu" "F.Paste" "F.Mask") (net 27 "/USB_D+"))
  (pad "5" smd rect (at 0 -1.15 270) (size 0.6 1.2) (layers "F.Cu" "F.Paste" "F.Mask") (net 4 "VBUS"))
  (pad "6" smd rect (at -0.95 -1.15 270) (size 0.6 1.2) (layers "F.Cu" "F.Paste" "F.Mask") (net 26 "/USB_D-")))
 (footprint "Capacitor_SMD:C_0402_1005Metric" (layer "F.Cu") (at 52.578 109.4285 180)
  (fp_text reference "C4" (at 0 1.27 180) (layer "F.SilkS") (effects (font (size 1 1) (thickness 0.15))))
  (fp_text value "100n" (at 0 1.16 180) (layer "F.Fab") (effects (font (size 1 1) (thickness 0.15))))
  (pad "1" smd roundrect (at -0.48 0 180) (size 0.56 0.62) (layers "F.Cu" "F.Paste" "F.Mask") (roundrect_rratio 0.25) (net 2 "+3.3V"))
  (pad "2" smd roundrect (at 0.48 0 180) (size 0.56 0.62) (layers "F.Cu" "F.Paste" "F.Mask") (roundrect_rratio 0.25) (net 1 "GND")))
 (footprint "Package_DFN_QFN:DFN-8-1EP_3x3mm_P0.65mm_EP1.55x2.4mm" (layer "F.Cu") (at 46.7425 113.63 180)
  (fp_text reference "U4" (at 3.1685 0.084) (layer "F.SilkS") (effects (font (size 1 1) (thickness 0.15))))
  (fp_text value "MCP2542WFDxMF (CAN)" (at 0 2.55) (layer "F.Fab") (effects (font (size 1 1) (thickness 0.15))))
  (pad "" smd rect (at -0.3875 -0.6 180) (size 0.6 1) (layers "F.Paste"))
  (pad "" smd rect (at -0.3875 0.6 180) (size 0.6 1) (layers "F.Paste"))
  (pad "" smd rect (at 0.3875 -0.6 180) (size 0.6 1) (layers "F.Paste"))
  (pad "" smd rect (at 0.3875 0.6 180) (size 0.6 1) (layers "F.Paste"))
  (pad "1" smd rect (at -1.55 -0.975 180) (size 0.65 0.35) (layers "F.Cu" "F.Paste" "F.Mask") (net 25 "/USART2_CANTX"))
  (pad "2" smd rect (at -1.55 -0.325 180) (size 0.65 0.35) (layers "F.Cu" "F.Paste" "F.Mask") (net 1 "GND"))
  (pad "3" smd rect (at -1.55 0.325 180) (size 0.65 0.35) (layers "F.Cu" "F.Paste" "F.Mask") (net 2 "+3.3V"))
  (pad "4" smd rect (at -1.55 0.975 180) (size 0.65 0.35) (layers "F.Cu" "F.Paste" "F.Mask") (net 24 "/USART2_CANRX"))
  (pad "5" smd rect (at 1.55 0.975 180) (size 0.65 0.35) (layers "F.Cu" "F.Paste" "F.Mask") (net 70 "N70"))
  (pad "6" smd rect (at 1.55 0.325 180) (size 0.65 0.35) (layers "F.Cu" "F.Paste" "F.Mask") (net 37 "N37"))
  (pad "7" smd rect (at 1.55 -0.325 180) (size 0.65 0.35) (layers "F.Cu" "F.Paste" "F.Mask") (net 35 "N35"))
  (pad "8" smd rect (at 1.55 -0.975 180) (size 0.65 0.35) (layers "F.Cu" "F.Paste" "F.Mask") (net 23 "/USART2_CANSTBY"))
  (pad "9" smd rect (at 0 0 180) (size 1.55 2.4) (layers "F.Cu" "F.Mask") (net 1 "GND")))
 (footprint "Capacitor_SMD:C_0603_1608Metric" (layer "F.Cu") (at 56.248 105.029)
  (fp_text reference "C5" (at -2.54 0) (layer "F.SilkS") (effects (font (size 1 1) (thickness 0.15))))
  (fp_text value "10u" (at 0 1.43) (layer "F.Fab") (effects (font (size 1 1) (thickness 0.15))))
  (pad "1" smd roundrect (at -0.775 0) (size 0.9 0.95) (layers "F.Cu" "F.Paste" "F.Mask") (roundrect_rratio 0.25) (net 2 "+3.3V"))
  (pad "2" smd roundrect (at 0.775 0) (size 0.9 0.95) (layers "F.Cu" "F.Paste" "F.Mask") (roundrect_rratio 0.25) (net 1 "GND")))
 (gr_rect (start 33.274 95.123) (end 91.186 124.46) (stroke (width 0.1) (type default)) (fill none) (layer "Edge.Cuts"))
 (via (at 41.529 100.711) (size 0.8) (drill 0.4) (layers "F.Cu" "B.Cu") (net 1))
 (via (at 41.529 99.187) (size 0.8) (drill 0.4) (layers "F.Cu" "B.Cu") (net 1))
 (via (at 39.116 102.489) (size 0.8) (drill 0.4) (layers "F.Cu" "B.Cu") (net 1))
 (via (at 41.529 97.282) (size 0.8) (drill 0.4) (layers "F.Cu" "B.Cu") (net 1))
 (via (at 39.116 97.282) (size 0.8) (drill 0.4) (layers "F.Cu" "B.Cu") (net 1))
 (via (at 43.688 99.187) (size 0.8) (drill 0.4) (layers "F.Cu" "B.Cu") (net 1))
 (via (at 39.116 99.187) (size 0.8) (drill 0.4) (layers "F.Cu" "B.Cu") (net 1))
 (via (at 43.688 100.838) (size 0.8) (drill 0.4) (layers "F.Cu" "B.Cu") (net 1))
 (via (at 39.116 100.838) (size 0.8) (drill 0.4) (layers "F.Cu" "B.Cu") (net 1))
 (via (at 43.688 97.282) (size 0.8) (drill 0.4) (layers "F.Cu" "B.Cu") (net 1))
 (via (at 41.529 102.489) (size 0.8) (drill 0.4) (layers "F.Cu" "B.Cu") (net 1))
 (via (at 43.688 102.489) (size 0.8) (drill 0.4) (layers "F.Cu" "B.Cu") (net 1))
 (segment (start 43.796999 116.652) (end 44.697 116.652) (width 0.2) (layer "F.Cu") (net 41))
 (segment (start 41.514 119.292499) (end 41.614 119.192499) (width 0.2) (layer "F.Cu") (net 41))
 (segment (start 43.071999 117.377) (end 43.796999 116.652) (width 0.2) (layer "F.Cu") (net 41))
 (segment (start 42.4518 117.377) (end 43.071999 117.377) (width 0.2) (layer "F.Cu") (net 41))
 (segment (start 41.514 120.305) (end 41.514 119.292499) (width 0.2) (layer "F.Cu") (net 41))
 (segment (start 41.614 118.2148) (end 42.4518 117.377) (width 0.2) (layer "F.Cu") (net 41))
 (segment (start 41.614 119.192499) (end 41.614 118.2148) (width 0.2) (layer "F.Cu") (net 41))
 (segment (start 42.164 119.292499) (end 42.064 119.192499) (width 0.2) (layer "F.Cu") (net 42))
 (segment (start 42.064 118.4012) (end 42.6382 117.827) (width 0.2) (layer "F.Cu") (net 42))
 (segment (start 42.6382 117.827) (end 43.071999 117.827) (width 0.2) (layer "F.Cu") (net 42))
 (segment (start 43.071999 117.827) (end 43.796999 118.552) (width 0.2) (layer "F.Cu") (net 42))
 (segment (start 42.164 120.305) (end 42.164 119.292499) (width 0.2) (layer "F.Cu") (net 42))
 (segment (start 42.064 119.192499) (end 42.064 118.4012) (width 0.2) (layer "F.Cu") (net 42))
 (segment (start 43.796999 118.552) (end 44.697 118.552) (width 0.2) (layer "F.Cu") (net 42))
 (segment (start 47.897001 118.552) (end 46.997 118.552) (width 0.2) (layer "F.Cu") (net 27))
 (segment (start 52.6712 117.827) (end 48.622001 117.827) (width 0.2) (layer "F.Cu") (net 27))
 (segment (start 53.565 113.6312) (end 53.565 116.9332) (width 0.2) (layer "F.Cu") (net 27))
 (segment (start 53.565 116.9332) (end 52.6712 117.827) (width 0.2) (layer "F.Cu") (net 27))
 (segment (start 56.1095 112.122) (end 55.453249 112.122) (width 0.2) (layer "F.Cu") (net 27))
 (segment (start 48.622001 117.827) (end 47.897001 118.552) (width 0.2) (layer "F.Cu") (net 27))
 (segment (start 55.453249 112.122) (end 55.428249 112.097) (width 0.2) (layer "F.Cu") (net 27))
 (segment (start 55.428249 112.097) (end 55.0992 112.097) (width 0.2) (layer "F.Cu") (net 27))
 (segment (start 55.0992 112.097) (end 53.565 113.6312) (width 0.2) (layer "F.Cu") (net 27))
 (segment (start 47.897001 116.652) (end 46.997 116.652) (width 0.2) (layer "F.Cu") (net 26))
 (segment (start 48.622001 117.377) (end 47.897001 116.652) (width 0.2) (layer "F.Cu") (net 26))
 (segment (start 53.115 113.4448) (end 53.115 116.7468) (width 0.2) (layer "F.Cu") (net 26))
 (segment (start 55.428249 111.647) (end 54.9128 111.647) (width 0.2) (layer "F.Cu") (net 26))
 (segment (start 52.4848 117.377) (end 48.622001 117.377) (width 0.2) (layer "F.Cu") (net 26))
 (segment (start 53.115 116.7468) (end 52.4848 117.377) (width 0.2) (layer "F.Cu") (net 26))
 (segment (start 54.9128 111.647) (end 53.115 113.4448) (width 0.2) (layer "F.Cu") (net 26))
 (segment (start 55.453249 111.622) (end 55.428249 111.647) (width 0.2) (layer "F.Cu") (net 26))
 (segment (start 56.1095 111.622) (end 55.453249 111.622) (width 0.2) (layer "F.Cu") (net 26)))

